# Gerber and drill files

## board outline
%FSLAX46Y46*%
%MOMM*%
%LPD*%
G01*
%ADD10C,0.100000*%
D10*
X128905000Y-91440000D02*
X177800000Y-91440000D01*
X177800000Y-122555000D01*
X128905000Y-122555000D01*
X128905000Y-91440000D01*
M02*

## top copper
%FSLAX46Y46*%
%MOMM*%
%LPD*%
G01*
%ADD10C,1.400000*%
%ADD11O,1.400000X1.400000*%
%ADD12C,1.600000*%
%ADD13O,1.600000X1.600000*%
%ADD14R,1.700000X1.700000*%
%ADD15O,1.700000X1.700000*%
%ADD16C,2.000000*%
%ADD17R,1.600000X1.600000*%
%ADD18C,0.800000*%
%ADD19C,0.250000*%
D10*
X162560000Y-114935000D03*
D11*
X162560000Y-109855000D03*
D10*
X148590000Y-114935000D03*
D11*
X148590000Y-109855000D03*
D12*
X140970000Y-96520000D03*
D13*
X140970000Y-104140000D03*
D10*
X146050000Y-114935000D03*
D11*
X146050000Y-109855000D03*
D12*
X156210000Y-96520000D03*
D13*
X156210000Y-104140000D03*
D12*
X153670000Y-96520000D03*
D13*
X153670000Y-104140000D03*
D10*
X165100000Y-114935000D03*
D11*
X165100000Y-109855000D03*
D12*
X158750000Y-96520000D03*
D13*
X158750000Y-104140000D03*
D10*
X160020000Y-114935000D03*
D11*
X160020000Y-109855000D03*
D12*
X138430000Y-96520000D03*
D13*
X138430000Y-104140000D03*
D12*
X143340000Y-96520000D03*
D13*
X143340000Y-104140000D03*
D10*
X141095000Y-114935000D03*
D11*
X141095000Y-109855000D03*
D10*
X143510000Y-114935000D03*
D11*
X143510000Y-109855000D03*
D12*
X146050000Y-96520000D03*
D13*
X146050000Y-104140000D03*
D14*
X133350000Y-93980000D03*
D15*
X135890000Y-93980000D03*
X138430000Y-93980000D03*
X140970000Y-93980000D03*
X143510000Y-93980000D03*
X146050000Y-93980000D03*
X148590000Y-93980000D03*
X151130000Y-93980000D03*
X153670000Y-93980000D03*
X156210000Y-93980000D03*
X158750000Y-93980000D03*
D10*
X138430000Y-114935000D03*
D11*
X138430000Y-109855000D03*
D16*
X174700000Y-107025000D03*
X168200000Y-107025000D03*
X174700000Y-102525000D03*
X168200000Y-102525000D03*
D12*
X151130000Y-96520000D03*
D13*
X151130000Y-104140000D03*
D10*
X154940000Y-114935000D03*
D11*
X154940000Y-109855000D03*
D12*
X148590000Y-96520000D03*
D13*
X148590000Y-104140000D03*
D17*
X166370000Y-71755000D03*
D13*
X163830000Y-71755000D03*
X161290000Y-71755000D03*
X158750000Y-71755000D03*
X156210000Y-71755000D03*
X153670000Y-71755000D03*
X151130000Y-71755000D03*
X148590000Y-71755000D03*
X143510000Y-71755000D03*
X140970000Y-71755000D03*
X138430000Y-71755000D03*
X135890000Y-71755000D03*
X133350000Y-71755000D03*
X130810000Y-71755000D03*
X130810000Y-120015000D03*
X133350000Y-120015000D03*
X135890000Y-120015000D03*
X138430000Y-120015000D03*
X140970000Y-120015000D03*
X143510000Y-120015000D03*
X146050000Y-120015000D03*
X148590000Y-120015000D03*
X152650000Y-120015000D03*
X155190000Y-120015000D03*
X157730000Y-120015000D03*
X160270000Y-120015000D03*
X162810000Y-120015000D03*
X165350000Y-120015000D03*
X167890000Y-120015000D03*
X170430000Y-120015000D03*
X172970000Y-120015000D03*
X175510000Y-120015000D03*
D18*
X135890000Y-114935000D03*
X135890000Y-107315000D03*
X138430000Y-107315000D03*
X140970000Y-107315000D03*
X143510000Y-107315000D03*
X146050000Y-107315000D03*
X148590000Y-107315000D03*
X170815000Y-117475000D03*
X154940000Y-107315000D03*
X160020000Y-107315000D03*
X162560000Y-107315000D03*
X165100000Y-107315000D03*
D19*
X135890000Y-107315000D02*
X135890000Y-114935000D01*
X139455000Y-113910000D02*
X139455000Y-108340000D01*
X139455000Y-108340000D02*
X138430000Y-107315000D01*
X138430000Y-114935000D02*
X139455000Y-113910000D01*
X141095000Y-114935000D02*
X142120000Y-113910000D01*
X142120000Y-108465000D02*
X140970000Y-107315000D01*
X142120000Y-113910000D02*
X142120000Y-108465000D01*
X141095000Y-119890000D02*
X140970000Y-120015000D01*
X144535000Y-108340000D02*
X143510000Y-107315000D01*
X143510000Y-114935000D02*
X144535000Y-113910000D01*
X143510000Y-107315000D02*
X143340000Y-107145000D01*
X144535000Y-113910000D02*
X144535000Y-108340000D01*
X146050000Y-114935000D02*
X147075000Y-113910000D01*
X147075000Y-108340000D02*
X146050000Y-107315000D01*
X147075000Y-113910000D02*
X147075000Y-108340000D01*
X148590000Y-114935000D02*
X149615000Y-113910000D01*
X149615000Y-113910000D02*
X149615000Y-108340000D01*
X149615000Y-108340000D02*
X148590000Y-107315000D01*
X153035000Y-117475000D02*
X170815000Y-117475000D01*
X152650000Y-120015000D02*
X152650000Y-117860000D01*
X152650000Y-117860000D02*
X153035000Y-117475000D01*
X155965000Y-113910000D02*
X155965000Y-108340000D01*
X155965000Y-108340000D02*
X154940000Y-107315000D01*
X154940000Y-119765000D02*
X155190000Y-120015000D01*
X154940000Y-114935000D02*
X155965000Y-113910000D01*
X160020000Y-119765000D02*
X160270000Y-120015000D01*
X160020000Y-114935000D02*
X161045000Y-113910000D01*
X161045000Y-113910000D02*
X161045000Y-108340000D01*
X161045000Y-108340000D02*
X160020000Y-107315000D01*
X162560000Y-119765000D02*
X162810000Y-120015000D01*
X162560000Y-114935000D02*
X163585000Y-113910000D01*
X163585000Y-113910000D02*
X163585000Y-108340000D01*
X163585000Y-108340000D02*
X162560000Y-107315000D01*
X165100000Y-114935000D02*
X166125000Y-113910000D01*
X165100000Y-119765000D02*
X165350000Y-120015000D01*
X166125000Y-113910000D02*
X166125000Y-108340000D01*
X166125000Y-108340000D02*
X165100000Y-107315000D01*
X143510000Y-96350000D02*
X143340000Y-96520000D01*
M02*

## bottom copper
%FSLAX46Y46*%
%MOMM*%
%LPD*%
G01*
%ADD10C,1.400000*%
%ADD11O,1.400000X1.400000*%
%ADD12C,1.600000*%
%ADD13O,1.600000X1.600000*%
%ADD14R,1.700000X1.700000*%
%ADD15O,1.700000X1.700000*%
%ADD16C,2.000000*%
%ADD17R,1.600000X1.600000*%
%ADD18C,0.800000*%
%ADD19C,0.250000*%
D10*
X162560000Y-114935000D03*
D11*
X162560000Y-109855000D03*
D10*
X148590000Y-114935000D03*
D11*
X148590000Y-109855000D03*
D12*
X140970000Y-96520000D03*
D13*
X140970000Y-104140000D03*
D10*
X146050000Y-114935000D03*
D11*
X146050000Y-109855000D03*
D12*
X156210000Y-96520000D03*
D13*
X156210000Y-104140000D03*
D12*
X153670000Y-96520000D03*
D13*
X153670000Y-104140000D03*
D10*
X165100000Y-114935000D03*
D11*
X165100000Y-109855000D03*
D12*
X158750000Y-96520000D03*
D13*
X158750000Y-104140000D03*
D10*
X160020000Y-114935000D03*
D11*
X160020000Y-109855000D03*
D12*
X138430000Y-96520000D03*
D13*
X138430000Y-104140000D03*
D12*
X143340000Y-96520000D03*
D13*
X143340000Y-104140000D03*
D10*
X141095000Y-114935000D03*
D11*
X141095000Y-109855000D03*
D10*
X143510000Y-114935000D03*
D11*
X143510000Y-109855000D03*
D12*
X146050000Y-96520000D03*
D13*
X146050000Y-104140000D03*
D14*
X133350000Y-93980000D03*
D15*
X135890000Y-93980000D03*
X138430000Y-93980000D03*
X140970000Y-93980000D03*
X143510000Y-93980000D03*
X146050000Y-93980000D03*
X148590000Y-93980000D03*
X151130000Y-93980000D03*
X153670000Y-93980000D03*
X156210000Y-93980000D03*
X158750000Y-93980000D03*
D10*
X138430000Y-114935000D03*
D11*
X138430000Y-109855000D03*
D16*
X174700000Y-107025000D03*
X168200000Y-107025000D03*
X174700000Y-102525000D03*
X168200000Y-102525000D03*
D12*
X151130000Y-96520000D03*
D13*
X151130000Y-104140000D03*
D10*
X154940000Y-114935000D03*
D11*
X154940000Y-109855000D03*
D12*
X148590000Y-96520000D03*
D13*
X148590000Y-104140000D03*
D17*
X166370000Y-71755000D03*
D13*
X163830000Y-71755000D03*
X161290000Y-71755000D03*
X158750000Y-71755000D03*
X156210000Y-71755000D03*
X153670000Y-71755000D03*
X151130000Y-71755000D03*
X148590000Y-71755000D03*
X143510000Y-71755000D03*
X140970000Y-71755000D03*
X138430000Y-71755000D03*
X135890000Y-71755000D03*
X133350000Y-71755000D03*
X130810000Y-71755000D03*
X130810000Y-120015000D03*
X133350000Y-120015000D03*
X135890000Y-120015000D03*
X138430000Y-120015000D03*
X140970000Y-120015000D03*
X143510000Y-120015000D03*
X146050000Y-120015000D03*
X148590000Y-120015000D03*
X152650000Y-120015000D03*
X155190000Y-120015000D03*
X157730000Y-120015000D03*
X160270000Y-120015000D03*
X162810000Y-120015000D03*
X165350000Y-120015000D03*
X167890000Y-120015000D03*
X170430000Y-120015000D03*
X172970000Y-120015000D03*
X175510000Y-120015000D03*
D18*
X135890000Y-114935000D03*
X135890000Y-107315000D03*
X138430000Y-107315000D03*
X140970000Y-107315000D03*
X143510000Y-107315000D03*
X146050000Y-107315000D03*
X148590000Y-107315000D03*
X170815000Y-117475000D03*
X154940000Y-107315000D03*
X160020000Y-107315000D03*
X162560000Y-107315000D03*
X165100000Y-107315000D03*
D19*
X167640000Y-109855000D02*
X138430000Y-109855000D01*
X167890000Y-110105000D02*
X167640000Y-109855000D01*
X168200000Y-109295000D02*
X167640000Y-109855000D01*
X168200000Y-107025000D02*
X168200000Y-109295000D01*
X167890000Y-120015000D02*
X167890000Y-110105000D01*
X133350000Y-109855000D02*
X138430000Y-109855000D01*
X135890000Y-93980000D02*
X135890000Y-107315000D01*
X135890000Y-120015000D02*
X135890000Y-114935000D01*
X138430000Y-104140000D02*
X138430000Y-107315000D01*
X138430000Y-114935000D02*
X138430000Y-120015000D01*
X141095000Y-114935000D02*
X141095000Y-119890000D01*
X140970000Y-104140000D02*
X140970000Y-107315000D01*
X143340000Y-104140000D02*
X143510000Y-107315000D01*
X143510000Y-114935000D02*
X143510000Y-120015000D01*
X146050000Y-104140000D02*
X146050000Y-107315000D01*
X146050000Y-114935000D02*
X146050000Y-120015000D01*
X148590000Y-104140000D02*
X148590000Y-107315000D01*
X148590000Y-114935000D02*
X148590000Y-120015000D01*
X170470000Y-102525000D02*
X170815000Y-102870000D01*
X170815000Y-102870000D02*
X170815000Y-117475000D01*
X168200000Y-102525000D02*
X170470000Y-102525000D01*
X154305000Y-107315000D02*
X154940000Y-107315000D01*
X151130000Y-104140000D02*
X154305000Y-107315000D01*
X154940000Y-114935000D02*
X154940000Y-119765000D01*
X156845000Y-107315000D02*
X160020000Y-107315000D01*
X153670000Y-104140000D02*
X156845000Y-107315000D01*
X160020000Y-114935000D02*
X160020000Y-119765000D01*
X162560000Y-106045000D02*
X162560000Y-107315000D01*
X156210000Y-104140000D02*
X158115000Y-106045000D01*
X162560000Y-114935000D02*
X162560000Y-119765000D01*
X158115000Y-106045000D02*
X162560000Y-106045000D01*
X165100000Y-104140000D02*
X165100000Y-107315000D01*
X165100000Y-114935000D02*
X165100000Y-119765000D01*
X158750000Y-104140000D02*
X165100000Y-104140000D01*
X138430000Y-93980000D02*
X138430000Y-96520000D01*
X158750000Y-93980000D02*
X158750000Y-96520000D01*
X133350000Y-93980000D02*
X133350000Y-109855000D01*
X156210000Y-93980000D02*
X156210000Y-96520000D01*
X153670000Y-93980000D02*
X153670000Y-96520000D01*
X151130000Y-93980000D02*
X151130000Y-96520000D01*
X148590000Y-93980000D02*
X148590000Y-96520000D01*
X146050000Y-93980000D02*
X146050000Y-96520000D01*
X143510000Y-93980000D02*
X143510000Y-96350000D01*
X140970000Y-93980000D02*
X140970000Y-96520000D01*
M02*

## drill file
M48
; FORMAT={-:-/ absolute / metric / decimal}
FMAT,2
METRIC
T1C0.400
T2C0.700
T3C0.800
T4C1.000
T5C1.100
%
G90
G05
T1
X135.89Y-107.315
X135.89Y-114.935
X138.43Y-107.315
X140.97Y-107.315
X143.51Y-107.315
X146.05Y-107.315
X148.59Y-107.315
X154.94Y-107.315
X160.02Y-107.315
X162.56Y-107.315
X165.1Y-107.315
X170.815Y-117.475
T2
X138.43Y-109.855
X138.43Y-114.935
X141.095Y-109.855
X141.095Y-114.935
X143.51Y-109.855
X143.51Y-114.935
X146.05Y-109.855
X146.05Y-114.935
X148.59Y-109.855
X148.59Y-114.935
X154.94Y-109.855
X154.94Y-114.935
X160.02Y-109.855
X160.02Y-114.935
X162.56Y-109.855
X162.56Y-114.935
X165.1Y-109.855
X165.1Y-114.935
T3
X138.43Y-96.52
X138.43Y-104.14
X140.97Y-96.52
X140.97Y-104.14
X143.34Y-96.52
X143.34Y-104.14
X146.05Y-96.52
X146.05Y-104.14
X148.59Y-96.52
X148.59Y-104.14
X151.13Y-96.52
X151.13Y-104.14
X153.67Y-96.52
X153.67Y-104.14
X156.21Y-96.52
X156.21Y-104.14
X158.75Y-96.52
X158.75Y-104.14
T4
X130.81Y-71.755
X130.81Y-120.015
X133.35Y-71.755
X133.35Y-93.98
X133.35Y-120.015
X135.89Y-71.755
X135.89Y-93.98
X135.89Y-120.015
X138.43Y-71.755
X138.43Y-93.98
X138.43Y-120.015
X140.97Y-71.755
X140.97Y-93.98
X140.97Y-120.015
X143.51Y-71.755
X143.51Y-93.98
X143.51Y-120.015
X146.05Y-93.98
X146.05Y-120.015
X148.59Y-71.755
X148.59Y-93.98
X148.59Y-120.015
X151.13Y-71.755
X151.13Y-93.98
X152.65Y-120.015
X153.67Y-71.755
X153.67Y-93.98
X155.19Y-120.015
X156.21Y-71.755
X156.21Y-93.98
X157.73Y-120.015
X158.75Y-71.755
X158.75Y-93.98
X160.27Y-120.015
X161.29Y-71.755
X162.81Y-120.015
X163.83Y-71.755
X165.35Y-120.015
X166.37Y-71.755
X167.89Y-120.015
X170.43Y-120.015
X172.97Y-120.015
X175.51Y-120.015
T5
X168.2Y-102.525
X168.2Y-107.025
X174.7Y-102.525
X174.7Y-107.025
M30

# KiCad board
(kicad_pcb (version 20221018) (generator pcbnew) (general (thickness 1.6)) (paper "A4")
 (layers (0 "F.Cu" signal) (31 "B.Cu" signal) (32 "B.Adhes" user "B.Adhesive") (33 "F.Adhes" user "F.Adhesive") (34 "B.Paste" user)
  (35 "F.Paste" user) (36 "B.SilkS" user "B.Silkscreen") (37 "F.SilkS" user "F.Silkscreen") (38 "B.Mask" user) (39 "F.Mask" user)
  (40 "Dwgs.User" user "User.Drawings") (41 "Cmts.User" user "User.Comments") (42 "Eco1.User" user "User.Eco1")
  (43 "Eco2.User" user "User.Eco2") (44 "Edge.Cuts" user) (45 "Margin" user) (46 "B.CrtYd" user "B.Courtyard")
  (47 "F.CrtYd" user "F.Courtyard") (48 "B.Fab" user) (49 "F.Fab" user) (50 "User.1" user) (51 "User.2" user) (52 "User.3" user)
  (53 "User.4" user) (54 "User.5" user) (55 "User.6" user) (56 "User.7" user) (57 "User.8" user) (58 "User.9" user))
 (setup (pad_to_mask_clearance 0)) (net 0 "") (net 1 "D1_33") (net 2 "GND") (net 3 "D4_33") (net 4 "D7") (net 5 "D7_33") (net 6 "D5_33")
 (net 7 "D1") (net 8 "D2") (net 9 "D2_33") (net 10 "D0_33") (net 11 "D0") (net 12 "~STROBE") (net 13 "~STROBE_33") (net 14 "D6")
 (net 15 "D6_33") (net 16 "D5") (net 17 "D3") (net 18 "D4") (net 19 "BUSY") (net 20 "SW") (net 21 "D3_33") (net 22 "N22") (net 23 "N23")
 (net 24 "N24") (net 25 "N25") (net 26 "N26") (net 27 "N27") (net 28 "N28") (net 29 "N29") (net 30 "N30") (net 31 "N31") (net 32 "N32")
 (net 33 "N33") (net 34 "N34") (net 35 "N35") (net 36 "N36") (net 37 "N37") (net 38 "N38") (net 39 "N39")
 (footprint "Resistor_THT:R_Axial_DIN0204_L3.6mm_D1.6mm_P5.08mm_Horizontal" (layer "F.Cu") (at 162.56 114.935 90)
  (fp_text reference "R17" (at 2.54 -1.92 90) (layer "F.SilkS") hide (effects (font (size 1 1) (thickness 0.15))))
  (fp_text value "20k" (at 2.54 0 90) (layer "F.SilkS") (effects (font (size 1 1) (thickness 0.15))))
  (pad "1" thru_hole circle (at 0 0 90) (size 1.4 1.4) (drill 0.7) (layers "*.Cu" "*.Mask") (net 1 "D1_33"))
  (pad "2" thru_hole oval (at 5.08 0 90) (size 1.4 1.4) (drill 0.7) (layers "*.Cu" "*.Mask") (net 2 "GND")))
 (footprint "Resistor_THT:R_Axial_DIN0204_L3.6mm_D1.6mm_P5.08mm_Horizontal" (layer "F.Cu") (at 148.59 114.935 90)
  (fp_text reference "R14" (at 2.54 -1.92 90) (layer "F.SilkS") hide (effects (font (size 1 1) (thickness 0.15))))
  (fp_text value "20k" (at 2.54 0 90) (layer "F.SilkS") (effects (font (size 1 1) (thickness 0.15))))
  (pad "1" thru_hole circle (at 0 0 90) (size 1.4 1.4) (drill 0.7) (layers "*.Cu" "*.Mask") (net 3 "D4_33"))
  (pad "2" thru_hole oval (at 5.08 0 90) (size 1.4 1.4) (drill 0.7) (layers "*.Cu" "*.Mask") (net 2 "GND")))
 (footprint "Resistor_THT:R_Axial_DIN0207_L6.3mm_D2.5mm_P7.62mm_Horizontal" (layer "F.Cu") (at 140.97 96.52 -90)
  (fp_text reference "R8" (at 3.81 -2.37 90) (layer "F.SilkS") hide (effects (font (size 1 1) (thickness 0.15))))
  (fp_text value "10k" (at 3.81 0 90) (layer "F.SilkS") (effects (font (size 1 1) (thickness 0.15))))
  (pad "1" thru_hole circle (at 0 0 270) (size 1.6 1.6) (drill 0.8) (layers "*.Cu" "*.Mask") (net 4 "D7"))
  (pad "2" thru_hole oval (at 7.62 0 270) (size 1.6 1.6) (drill 0.8) (layers "*.Cu" "*.Mask") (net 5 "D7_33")))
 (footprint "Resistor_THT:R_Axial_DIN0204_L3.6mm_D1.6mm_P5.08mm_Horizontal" (layer "F.Cu") (at 146.05 114.935 90)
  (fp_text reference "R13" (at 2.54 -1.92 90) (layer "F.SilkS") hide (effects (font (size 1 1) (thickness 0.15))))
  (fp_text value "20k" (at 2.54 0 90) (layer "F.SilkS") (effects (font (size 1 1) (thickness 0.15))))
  (pad "1" thru_hole circle (at 0 0 90) (size 1.4 1.4) (drill 0.7) (layers "*.Cu" "*.Mask") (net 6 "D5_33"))
  (pad "2" thru_hole oval (at 5.08 0 90) (size 1.4 1.4) (drill 0.7) (layers "*.Cu" "*.Mask") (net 2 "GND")))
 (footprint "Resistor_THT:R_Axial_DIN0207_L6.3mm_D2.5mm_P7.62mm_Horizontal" (layer "F.Cu") (at 156.21 96.52 -90)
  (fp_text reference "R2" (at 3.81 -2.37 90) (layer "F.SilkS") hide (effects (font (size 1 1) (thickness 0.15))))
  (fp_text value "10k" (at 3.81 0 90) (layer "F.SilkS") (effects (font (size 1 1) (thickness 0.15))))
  (pad "1" thru_hole circle (at 0 0 270) (size 1.6 1.6) (drill 0.8) (layers "*.Cu" "*.Mask") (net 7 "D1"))
  (pad "2" thru_hole oval (at 7.62 0 270) (size 1.6 1.6) (drill 0.8) (layers "*.Cu" "*.Mask") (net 1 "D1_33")))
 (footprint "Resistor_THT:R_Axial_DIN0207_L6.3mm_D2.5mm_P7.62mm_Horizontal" (layer "F.Cu") (at 153.67 96.52 -90)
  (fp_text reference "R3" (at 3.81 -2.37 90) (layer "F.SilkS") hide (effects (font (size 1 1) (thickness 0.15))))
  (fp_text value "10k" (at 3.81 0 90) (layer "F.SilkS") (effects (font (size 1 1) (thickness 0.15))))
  (pad "1" thru_hole circle (at 0 0 270) (size 1.6 1.6) (drill 0.8) (layers "*.Cu" "*.Mask") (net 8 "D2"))
  (pad "2" thru_hole oval (at 7.62 0 270) (size 1.6 1.6) (drill 0.8) (layers "*.Cu" "*.Mask") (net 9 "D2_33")))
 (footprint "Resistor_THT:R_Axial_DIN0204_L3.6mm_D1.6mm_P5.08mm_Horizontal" (layer "F.Cu") (at 165.1 114.935 90)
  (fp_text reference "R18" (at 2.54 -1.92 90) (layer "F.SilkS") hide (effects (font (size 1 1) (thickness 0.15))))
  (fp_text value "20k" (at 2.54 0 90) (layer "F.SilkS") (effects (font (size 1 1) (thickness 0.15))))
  (pad "1" thru_hole circle (at 0 0 90) (size 1.4 1.4) (drill 0.7) (layers "*.Cu" "*.Mask") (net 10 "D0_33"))
  (pad "2" thru_hole oval (at 5.08 0 90) (size 1.4 1.4) (drill 0.7) (layers "*.Cu" "*.Mask") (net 2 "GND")))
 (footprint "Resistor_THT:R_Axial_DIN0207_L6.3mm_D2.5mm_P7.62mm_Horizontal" (layer "F.Cu") (at 158.75 96.52 -90)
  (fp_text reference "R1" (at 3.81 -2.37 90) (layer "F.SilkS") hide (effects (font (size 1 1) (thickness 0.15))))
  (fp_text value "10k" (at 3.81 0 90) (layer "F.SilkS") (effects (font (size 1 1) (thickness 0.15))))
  (pad "1" thru_hole circle (at 0 0 270) (size 1.6 1.6) (drill 0.8) (layers "*.Cu" "*.Mask") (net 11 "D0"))
  (pad "2" thru_hole oval (at 7.62 0 270) (size 1.6 1.6) (drill 0.8) (layers "*.Cu" "*.Mask") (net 10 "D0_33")))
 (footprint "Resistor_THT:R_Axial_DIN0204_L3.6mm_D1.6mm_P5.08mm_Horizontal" (layer "F.Cu") (at 160.02 114.935 90)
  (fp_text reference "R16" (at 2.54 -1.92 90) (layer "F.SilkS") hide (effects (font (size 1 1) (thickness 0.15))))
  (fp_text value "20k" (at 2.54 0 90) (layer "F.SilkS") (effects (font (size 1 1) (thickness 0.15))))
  (pad "1" thru_hole circle (at 0 0 90) (size 1.4 1.4) (drill 0.7) (layers "*.Cu" "*.Mask") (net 9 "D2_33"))
  (pad "2" thru_hole oval (at 5.08 0 90) (size 1.4 1.4) (drill 0.7) (layers "*.Cu" "*.Mask") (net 2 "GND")))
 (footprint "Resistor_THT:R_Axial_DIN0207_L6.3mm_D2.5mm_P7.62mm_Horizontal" (layer "F.Cu") (at 138.43 96.52 -90)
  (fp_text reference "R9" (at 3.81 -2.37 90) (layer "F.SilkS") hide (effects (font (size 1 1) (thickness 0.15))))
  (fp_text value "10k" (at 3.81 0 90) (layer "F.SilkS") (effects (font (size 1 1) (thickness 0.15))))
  (pad "1" thru_hole circle (at 0 0 270) (size 1.6 1.6) (drill 0.8) (layers "*.Cu" "*.Mask") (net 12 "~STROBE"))
  (pad "2" thru_hole oval (at 7.62 0 270) (size 1.6 1.6) (drill 0.8) (layers "*.Cu" "*.Mask") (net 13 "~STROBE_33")))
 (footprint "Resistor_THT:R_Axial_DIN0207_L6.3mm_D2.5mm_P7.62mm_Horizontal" (layer "F.Cu") (at 143.34 96.52 -90)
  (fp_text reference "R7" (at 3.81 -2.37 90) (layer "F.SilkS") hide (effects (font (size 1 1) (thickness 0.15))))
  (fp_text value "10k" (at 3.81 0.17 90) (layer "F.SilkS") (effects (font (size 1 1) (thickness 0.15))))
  (pad "1" thru_hole circle (at 0 0 270) (size 1.6 1.6) (drill 0.8) (layers "*.Cu" "*.Mask") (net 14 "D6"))
  (pad "2" thru_hole oval (at 7.62 0 270) (size 1.6 1.6) (drill 0.8) (layers "*.Cu" "*.Mask") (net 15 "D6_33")))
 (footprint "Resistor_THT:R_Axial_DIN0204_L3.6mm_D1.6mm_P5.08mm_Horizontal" (layer "F.Cu") (at 141.095 114.935 90)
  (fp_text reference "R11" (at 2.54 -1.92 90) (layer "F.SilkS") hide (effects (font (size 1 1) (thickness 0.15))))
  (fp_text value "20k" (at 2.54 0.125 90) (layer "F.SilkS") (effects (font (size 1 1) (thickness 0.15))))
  (pad "1" thru_hole circle (at 0 0 90) (size 1.4 1.4) (drill 0.7) (layers "*.Cu" "*.Mask") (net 5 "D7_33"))
  (pad "2" thru_hole oval (at 5.08 0 90) (size 1.4 1.4) (drill 0.7) (layers "*.Cu" "*.Mask") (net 2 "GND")))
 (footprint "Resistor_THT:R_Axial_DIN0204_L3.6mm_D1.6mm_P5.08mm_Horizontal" (layer "F.Cu") (at 143.51 114.935 90)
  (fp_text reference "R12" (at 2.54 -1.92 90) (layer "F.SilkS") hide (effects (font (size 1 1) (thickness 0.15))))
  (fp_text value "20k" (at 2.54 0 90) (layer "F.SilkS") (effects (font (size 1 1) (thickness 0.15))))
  (pad "1" thru_hole circle (at 0 0 90) (size 1.4 1.4) (drill 0.7) (layers "*.Cu" "*.Mask") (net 15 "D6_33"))
  (pad "2" thru_hole oval (at 5.08 0 90) (size 1.4 1.4) (drill 0.7) (layers "*.Cu" "*.Mask") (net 2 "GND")))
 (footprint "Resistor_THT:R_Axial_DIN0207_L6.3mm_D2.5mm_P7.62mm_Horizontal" (layer "F.Cu") (at 146.05 96.52 -90)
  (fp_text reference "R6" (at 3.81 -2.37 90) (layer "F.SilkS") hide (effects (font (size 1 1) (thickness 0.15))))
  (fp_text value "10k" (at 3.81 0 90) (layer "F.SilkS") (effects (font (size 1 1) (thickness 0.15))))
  (pad "1" thru_hole circle (at 0 0 270) (size 1.6 1.6) (drill 0.8) (layers "*.Cu" "*.Mask") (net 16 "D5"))
  (pad "2" thru_hole oval (at 7.62 0 270) (size 1.6 1.6) (drill 0.8) (layers "*.Cu" "*.Mask") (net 6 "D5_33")))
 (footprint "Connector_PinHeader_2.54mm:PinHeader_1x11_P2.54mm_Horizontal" (layer "F.Cu") (at 133.35 93.98 90)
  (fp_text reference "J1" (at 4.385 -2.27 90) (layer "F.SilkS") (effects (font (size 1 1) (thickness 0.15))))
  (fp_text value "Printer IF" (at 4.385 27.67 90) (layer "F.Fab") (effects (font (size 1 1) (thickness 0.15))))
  (pad "1" thru_hole rect (at 0 0 90) (size 1.7 1.7) (drill 1) (layers "*.Cu" "*.Mask") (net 11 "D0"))
  (pad "2" thru_hole oval (at 0 2.54 90) (size 1.7 1.7) (drill 1) (layers "*.Cu" "*.Mask") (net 7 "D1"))
  (pad "3" thru_hole oval (at 0 5.08 90) (size 1.7 1.7) (drill 1) (layers "*.Cu" "*.Mask") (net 8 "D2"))
  (pad "4" thru_hole oval (at 0 7.62 90) (size 1.7 1.7) (drill 1) (layers "*.Cu" "*.Mask") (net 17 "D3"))
  (pad "5" thru_hole oval (at 0 10.16 90) (size 1.7 1.7) (drill 1) (layers "*.Cu" "*.Mask") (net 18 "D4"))
  (pad "6" thru_hole oval (at 0 12.7 90) (size 1.7 1.7) (drill 1) (layers "*.Cu" "*.Mask") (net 16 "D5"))
  (pad "7" thru_hole oval (at 0 15.24 90) (size 1.7 1.7) (drill 1) (layers "*.Cu" "*.Mask") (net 14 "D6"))
  (pad "8" thru_hole oval (at 0 17.78 90) (size 1.7 1.7) (drill 1) (layers "*.Cu" "*.Mask") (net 4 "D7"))
  (pad "9" thru_hole oval (at 0 20.32 90) (size 1.7 1.7) (drill 1) (layers "*.Cu" "*.Mask") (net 12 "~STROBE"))
  (pad "10" thru_hole oval (at 0 22.86 90) (size 1.7 1.7) (drill 1) (layers "*.Cu" "*.Mask") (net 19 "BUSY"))
  (pad "11" thru_hole oval (at 0 25.4 90) (size 1.7 1.7) (drill 1) (layers "*.Cu" "*.Mask") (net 2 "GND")))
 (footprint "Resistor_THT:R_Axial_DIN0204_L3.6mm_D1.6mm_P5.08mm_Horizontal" (layer "F.Cu") (at 138.43 114.935 90)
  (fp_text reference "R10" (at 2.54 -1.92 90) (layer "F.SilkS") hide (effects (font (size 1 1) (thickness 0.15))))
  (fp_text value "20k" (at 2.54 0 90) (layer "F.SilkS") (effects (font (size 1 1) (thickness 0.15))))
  (pad "1" thru_hole circle (at 0 0 90) (size 1.4 1.4) (drill 0.7) (layers "*.Cu" "*.Mask") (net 13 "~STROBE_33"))
  (pad "2" thru_hole oval (at 5.08 0 90) (size 1.4 1.4) (drill 0.7) (layers "*.Cu" "*.Mask") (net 2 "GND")))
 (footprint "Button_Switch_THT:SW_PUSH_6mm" (layer "F.Cu") (at 174.7 107.025 180)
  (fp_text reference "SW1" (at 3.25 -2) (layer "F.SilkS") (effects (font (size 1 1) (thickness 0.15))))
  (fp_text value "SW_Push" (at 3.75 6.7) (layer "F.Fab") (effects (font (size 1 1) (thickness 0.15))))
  (pad "1" thru_hole circle (at 0 0 270) (size 2 2) (drill 1.1) (layers "*.Cu" "*.Mask") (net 2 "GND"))
  (pad "1" thru_hole circle (at 6.5 0 270) (size 2 2) (drill 1.1) (layers "*.Cu" "*.Mask") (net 2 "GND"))
  (pad "2" thru_hole circle (at 0 4.5 270) (size 2 2) (drill 1.1) (layers "*.Cu" "*.Mask") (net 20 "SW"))
  (pad "2" thru_hole circle (at 6.5 4.5 270) (size 2 2) (drill 1.1) (layers "*.Cu" "*.Mask") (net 20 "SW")))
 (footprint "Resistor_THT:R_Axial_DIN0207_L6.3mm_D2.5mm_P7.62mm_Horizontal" (layer "F.Cu") (at 151.13 96.52 -90)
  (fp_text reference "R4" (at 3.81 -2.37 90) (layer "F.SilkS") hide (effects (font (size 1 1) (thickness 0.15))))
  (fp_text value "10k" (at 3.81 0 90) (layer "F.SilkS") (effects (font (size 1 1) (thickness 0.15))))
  (pad "1" thru_hole circle (at 0 0 270) (size 1.6 1.6) (drill 0.8) (layers "*.Cu" "*.Mask") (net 17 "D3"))
  (pad "2" thru_hole oval (at 7.62 0 270) (size 1.6 1.6) (drill 0.8) (layers "*.Cu" "*.Mask") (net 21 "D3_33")))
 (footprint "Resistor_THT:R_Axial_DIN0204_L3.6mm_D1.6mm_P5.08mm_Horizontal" (layer "F.Cu") (at 154.94 114.935 90)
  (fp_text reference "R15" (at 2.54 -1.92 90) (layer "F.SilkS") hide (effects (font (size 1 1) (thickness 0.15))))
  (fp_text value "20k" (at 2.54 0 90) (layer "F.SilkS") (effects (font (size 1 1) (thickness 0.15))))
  (pad "1" thru_hole circle (at 0 0 90) (size 1.4 1.4) (drill 0.7) (layers "*.Cu" "*.Mask") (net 21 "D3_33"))
  (pad "2" thru_hole oval (at 5.08 0 90) (size 1.4 1.4) (drill 0.7) (layers "*.Cu" "*.Mask") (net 2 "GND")))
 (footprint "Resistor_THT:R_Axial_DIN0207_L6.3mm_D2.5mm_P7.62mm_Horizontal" (layer "F.Cu") (at 148.59 96.52 -90)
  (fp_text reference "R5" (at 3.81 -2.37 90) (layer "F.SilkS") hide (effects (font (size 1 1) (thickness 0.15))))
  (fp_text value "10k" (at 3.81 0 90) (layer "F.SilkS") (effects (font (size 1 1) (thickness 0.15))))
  (pad "1" thru_hole circle (at 0 0 270) (size 1.6 1.6) (drill 0.8) (layers "*.Cu" "*.Mask") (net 18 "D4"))
  (pad "2" thru_hole oval (at 7.62 0 270) (size 1.6 1.6) (drill 0.8) (layers "*.Cu" "*.Mask") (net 3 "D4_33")))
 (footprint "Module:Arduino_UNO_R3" (layer "B.Cu") (at 166.37 71.755 180)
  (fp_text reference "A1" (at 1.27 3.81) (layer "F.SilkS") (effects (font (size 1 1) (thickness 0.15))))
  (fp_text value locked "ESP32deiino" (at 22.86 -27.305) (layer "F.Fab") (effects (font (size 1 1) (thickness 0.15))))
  (pad "1" thru_hole rect (at 0 0 90) (size 1.6 1.6) (drill 1) (layers "*.Cu" "*.Mask") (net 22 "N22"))
  (pad "2" thru_hole oval (at 2.54 0 90) (size 1.6 1.6) (drill 1) (layers "*.Cu" "*.Mask") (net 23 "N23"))
  (pad "3" thru_hole oval (at 5.08 0 90) (size 1.6 1.6) (drill 1) (layers "*.Cu" "*.Mask") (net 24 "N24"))
  (pad "4" thru_hole oval (at 7.62 0 90) (size 1.6 1.6) (drill 1) (layers "*.Cu" "*.Mask") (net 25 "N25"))
  (pad "5" thru_hole oval (at 10.16 0 90) (size 1.6 1.6) (drill 1) (layers "*.Cu" "*.Mask") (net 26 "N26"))
  (pad "6" thru_hole oval (at 12.7 0 90) (size 1.6 1.6) (drill 1) (layers "*.Cu" "*.Mask") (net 2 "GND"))
  (pad "7" thru_hole oval (at 15.24 0 90) (size 1.6 1.6) (drill 1) (layers "*.Cu" "*.Mask") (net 2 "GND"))
  (pad "8" thru_hole oval (at 17.78 0 90) (size 1.6 1.6) (drill 1) (layers "*.Cu" "*.Mask") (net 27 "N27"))
  (pad "9" thru_hole oval (at 22.86 0 90) (size 1.6 1.6) (drill 1) (layers "*.Cu" "*.Mask") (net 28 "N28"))
  (pad "10" thru_hole oval (at 25.4 0 90) (size 1.6 1.6) (drill 1) (layers "*.Cu" "*.Mask") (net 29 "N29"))
  (pad "11" thru_hole oval (at 27.94 0 90) (size 1.6 1.6) (drill 1) (layers "*.Cu" "*.Mask") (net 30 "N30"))
  (pad "12" thru_hole oval (at 30.48 0 90) (size 1.6 1.6) (drill 1) (layers "*.Cu" "*.Mask") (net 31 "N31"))
  (pad "13" thru_hole oval (at 33.02 0 90) (size 1.6 1.6) (drill 1) (layers "*.Cu" "*.Mask") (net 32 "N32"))
  (pad "14" thru_hole oval (at 35.56 0 90) (size 1.6 1.6) (drill 1) (layers "*.Cu" "*.Mask") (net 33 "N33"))
  (pad "15" thru_hole oval (at 35.56 -48.26 90) (size 1.6 1.6) (drill 1) (layers "*.Cu" "*.Mask") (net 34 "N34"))
  (pad "16" thru_hole oval (at 33.02 -48.26 90) (size 1.6 1.6) (drill 1) (layers "*.Cu" "*.Mask") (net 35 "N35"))
  (pad "17" thru_hole oval (at 30.48 -48.26 90) (size 1.6 1.6) (drill 1) (layers "*.Cu" "*.Mask") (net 19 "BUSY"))
  (pad "18" thru_hole oval (at 27.94 -48.26 90) (size 1.6 1.6) (drill 1) (layers "*.Cu" "*.Mask") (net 13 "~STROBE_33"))
  (pad "19" thru_hole oval (at 25.4 -48.26 90) (size 1.6 1.6) (drill 1) (layers "*.Cu" "*.Mask") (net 5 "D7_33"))
  (pad "20" thru_hole oval (at 22.86 -48.26 90) (size 1.6 1.6) (drill 1) (layers "*.Cu" "*.Mask") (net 15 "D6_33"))
  (pad "21" thru_hole oval (at 20.32 -48.26 90) (size 1.6 1.6) (drill 1) (layers "*.Cu" "*.Mask") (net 6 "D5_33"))
  (pad "22" thru_hole oval (at 17.78 -48.26 90) (size 1.6 1.6) (drill 1) (layers "*.Cu" "*.Mask") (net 3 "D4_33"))
  (pad "23" thru_hole oval (at 13.72 -48.26 90) (size 1.6 1.6) (drill 1) (layers "*.Cu" "*.Mask") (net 20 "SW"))
  (pad "24" thru_hole oval (at 11.18 -48.26 90) (size 1.6 1.6) (drill 1) (layers "*.Cu" "*.Mask") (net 21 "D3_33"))
  (pad "25" thru_hole oval (at 8.64 -48.26 90) (size 1.6 1.6) (drill 1) (layers "*.Cu" "*.Mask") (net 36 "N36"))
  (pad "26" thru_hole oval (at 6.1 -48.26 90) (size 1.6 1.6) (drill 1) (layers "*.Cu" "*.Mask") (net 9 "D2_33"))
  (pad "27" thru_hole oval (at 3.56 -48.26 90) (size 1.6 1.6) (drill 1) (layers "*.Cu" "*.Mask") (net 1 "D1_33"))
  (pad "28" thru_hole oval (at 1.02 -48.26 90) (size 1.6 1.6) (drill 1) (layers "*.Cu" "*.Mask") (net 10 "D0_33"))
  (pad "29" thru_hole oval (at -1.52 -48.26 90) (size 1.6 1.6) (drill 1) (layers "*.Cu" "*.Mask") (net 2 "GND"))
  (pad "30" thru_hole oval (at -4.06 -48.26 90) (size 1.6 1.6) (drill 1) (layers "*.Cu" "*.Mask") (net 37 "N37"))
  (pad "31" thru_hole oval (at -6.6 -48.26 90) (size 1.6 1.6) (drill 1) (layers "*.Cu" "*.Mask") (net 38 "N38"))
  (pad "32" thru_hole oval (at -9.14 -48.26 90) (size 1.6 1.6) (drill 1) (layers "*.Cu" "*.Mask") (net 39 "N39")))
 (gr_rect (start 128.905 91.44) (end 177.8 122.555) (stroke (width 0.1) (type default)) (fill none) (layer "Edge.Cuts"))
 (segment (start 167.64 109.855) (end 138.43 109.855) (width 0.25) (layer "B.Cu") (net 2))
 (segment (start 167.89 110.105) (end 167.64 109.855) (width 0.25) (layer "B.Cu") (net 2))
 (segment (start 168.2 109.295) (end 167.64 109.855) (width 0.25) (layer "B.Cu") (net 2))
 (segment (start 168.2 107.025) (end 168.2 109.295) (width 0.25) (layer "B.Cu") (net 2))
 (segment (start 167.89 120.015) (end 167.89 110.105) (width 0.25) (layer "B.Cu") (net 2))
 (segment (start 133.35 109.855) (end 138.43 109.855) (width 0.25) (layer "B.Cu") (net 2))
 (segment (start 135.89 107.315) (end 135.89 114.935) (width 0.25) (layer "F.Cu") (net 19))
 (via (at 135.89 114.935) (size 0.8) (drill 0.4) (layers "F.Cu" "B.Cu") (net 19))
 (via (at 135.89 107.315) (size 0.8) (drill 0.4) (layers "F.Cu" "B.Cu") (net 19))
 (segment (start 135.89 93.98) (end 135.89 107.315) (width 0.25) (layer "B.Cu") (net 19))
 (segment (start 135.89 120.015) (end 135.89 114.935) (width 0.25) (layer "B.Cu") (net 19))
 (segment (start 139.455 113.91) (end 139.455 108.34) (width 0.25) (layer "F.Cu") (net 13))
 (segment (start 139.455 108.34) (end 138.43 107.315) (width 0.25) (layer "F.Cu") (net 13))
 (segment (start 138.43 114.935) (end 139.455 113.91) (width 0.25) (layer "F.Cu") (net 13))
 (via (at 138.43 107.315) (size 0.8) (drill 0.4) (layers "F.Cu" "B.Cu") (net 13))
 (segment (start 138.43 104.14) (end 138.43 107.315) (width 0.25) (layer "B.Cu") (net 13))
 (segment (start 138.43 114.935) (end 138.43 120.015) (width 0.25) (layer "B.Cu") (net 13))
 (segment (start 141.095 114.935) (end 142.12 113.91) (width 0.25) (layer "F.Cu") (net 5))
 (segment (start 142.12 108.465) (end 140.97 107.315) (width 0.25) (layer "F.Cu") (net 5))
 (segment (start 142.12 113.91) (end 142.12 108.465) (width 0.25) (layer "F.Cu") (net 5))
 (segment (start 141.095 119.89) (end 140.97 120.015) (width 0.25) (layer "F.Cu") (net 5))
 (via (at 140.97 107.315) (size 0.8) (drill 0.4) (layers "F.Cu" "B.Cu") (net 5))
 (segment (start 141.095 114.935) (end 141.095 119.89) (width 0.25) (layer "B.Cu") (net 5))
 (segment (start 140.97 104.14) (end 140.97 107.315) (width 0.25) (layer "B.Cu") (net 5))
 (segment (start 144.535 108.34) (end 143.51 107.315) (width 0.25) (layer "F.Cu") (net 15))
 (segment (start 143.51 114.935) (end 144.535 113.91) (width 0.25) (layer "F.Cu") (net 15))
 (segment (start 143.51 107.315) (end 143.34 107.145) (width 0.25) (layer "F.Cu") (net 15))
 (segment (start 144.535 113.91) (end 144.535 108.34) (width 0.25) (layer "F.Cu") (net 15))
 (via (at 143.51 107.315) (size 0.8) (drill 0.4) (layers "F.Cu" "B.Cu") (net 15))
 (segment (start 143.34 104.14) (end 143.51 107.315) (width 0.25) (layer "B.Cu") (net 15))
 (segment (start 143.51 114.935) (end 143.51 120.015) (width 0.25) (layer "B.Cu") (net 15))
 (segment (start 146.05 114.935) (end 147.075 113.91) (width 0.25) (layer "F.Cu") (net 6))
 (segment (start 147.075 108.34) (end 146.05 107.315) (width 0.25) (layer "F.Cu") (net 6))
 (segment (start 147.075 113.91) (end 147.075 108.34) (width 0.25) (layer "F.Cu") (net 6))
 (via (at 146.05 107.315) (size 0.8) (drill 0.4) (layers "F.Cu" "B.Cu") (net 6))
 (segment (start 146.05 104.14) (end 146.05 107.315) (width 0.25) (layer "B.Cu") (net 6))
 (segment (start 146.05 114.935) (end 146.05 120.015) (width 0.25) (layer "B.Cu") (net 6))
 (segment (start 148.59 114.935) (end 149.615 113.91) (width 0.25) (layer "F.Cu") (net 3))
 (segment (start 149.615 113.91) (end 149.615 108.34) (width 0.25) (layer "F.Cu") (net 3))
 (segment (start 149.615 108.34) (end 148.59 107.315) (width 0.25) (layer "F.Cu") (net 3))
 (via (at 148.59 107.315) (size 0.8) (drill 0.4) (layers "F.Cu" "B.Cu") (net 3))
 (segment (start 148.59 104.14) (end 148.59 107.315) (width 0.25) (layer "B.Cu") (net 3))
 (segment (start 148.59 114.935) (end 148.59 120.015) (width 0.25) (layer "B.Cu") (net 3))
 (segment (start 153.035 117.475) (end 170.815 117.475) (width 0.25) (layer "F.Cu") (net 20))
 (segment (start 152.65 120.015) (end 152.65 117.86) (width 0.25) (layer "F.Cu") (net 20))
 (segment (start 152.65 117.86) (end 153.035 117.475) (width 0.25) (layer "F.Cu") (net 20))
 (via (at 170.815 117.475) (size 0.8) (drill 0.4) (layers "F.Cu" "B.Cu") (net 20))
 (segment (start 170.47 102.525) (end 170.815 102.87) (width 0.25) (layer "B.Cu") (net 20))
 (segment (start 170.815 102.87) (end 170.815 117.475) (width 0.25) (layer "B.Cu") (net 20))
 (segment (start 168.2 102.525) (end 170.47 102.525) (width 0.25) (layer "B.Cu") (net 20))
 (segment (start 155.965 113.91) (end 155.965 108.34) (width 0.25) (layer "F.Cu") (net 21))
 (segment (start 155.965 108.34) (end 154.94 107.315) (width 0.25) (layer "F.Cu") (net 21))
 (segment (start 154.94 119.765) (end 155.19 120.015) (width 0.25) (layer "F.Cu") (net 21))
 (segment (start 154.94 114.935) (end 155.965 113.91) (width 0.25) (layer "F.Cu") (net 21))
 (via (at 154.94 107.315) (size 0.8) (drill 0.4) (layers "F.Cu" "B.Cu") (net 21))
 (segment (start 154.305 107.315) (end 154.94 107.315) (width 0.25) (layer "B.Cu") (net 21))
 (segment (start 151.13 104.14) (end 154.305 107.315) (width 0.25) (layer "B.Cu") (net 21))
 (segment (start 154.94 114.935) (end 154.94 119.765) (width 0.25) (layer "B.Cu") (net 21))
 (segment (start 160.02 119.765) (end 160.27 120.015) (width 0.25) (layer "F.Cu") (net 9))
 (segment (start 160.02 114.935) (end 161.045 113.91) (width 0.25) (layer "F.Cu") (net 9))
 (segment (start 161.045 113.91) (end 161.045 108.34) (width 0.25) (layer "F.Cu") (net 9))
 (segment (start 161.045 108.34) (end 160.02 107.315) (width 0.25) (layer "F.Cu") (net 9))
 (via (at 160.02 107.315) (size 0.8) (drill 0.4) (layers "F.Cu" "B.Cu") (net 9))
 (segment (start 156.845 107.315) (end 160.02 107.315) (width 0.25) (layer "B.Cu") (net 9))
 (segment (start 153.67 104.14) (end 156.845 107.315) (width 0.25) (layer "B.Cu") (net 9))
 (segment (start 160.02 114.935) (end 160.02 119.765) (width 0.25) (layer "B.Cu") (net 9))
 (segment (start 162.56 119.765) (end 162.81 120.015) (width 0.25) (layer "F.Cu") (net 1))
 (segment (start 162.56 114.935) (end 163.585 113.91) (width 0.25) (layer "F.Cu") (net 1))
 (segment (start 163.585 113.91) (end 163.585 108.34) (width 0.25) (layer "F.Cu") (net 1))
 (segment (start 163.585 108.34) (end 162.56 107.315) (width 0.25) (layer "F.Cu") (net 1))
 (via (at 162.56 107.315) (size 0.8) (drill 0.4) (layers "F.Cu" "B.Cu") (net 1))
 (segment (start 162.56 106.045) (end 162.56 107.315) (width 0.25) (layer "B.Cu") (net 1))
 (segment (start 156.21 104.14) (end 158.115 106.045) (width 0.25) (layer "B.Cu") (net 1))
 (segment (start 162.56 114.935) (end 162.56 119.765) (width 0.25) (layer "B.Cu") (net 1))
 (segment (start 158.115 106.045) (end 162.56 106.045) (width 0.25) (layer "B.Cu") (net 1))
 (segment (start 165.1 114.935) (end 166.125 113.91) (width 0.25) (layer "F.Cu") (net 10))
 (segment (start 165.1 119.765) (end 165.35 120.015) (width 0.25) (layer "F.Cu") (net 10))
 (segment (start 166.125 113.91) (end 166.125 108.34) (width 0.25) (layer "F.Cu") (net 10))
 (segment (start 166.125 108.34) (end 165.1 107.315) (width 0.25) (layer "F.Cu") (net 10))
 (via (at 165.1 107.315) (size 0.8) (drill 0.4) (layers "F.Cu" "B.Cu") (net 10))
 (segment (start 165.1 104.14) (end 165.1 107.315) (width 0.25) (layer "B.Cu") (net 10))
 (segment (start 165.1 114.935) (end 165.1 119.765) (width 0.25) (layer "B.Cu") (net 10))
 (segment (start 158.75 104.14) (end 165.1 104.14) (width 0.25) (layer "B.Cu") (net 10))
 (segment (start 138.43 93.98) (end 138.43 96.52) (width 0.25) (layer "B.Cu") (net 12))
 (segment (start 158.75 93.98) (end 158.75 96.52) (width 0.25) (layer "B.Cu") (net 11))
 (segment (start 133.35 93.98) (end 133.35 109.855) (width 0.25) (layer "B.Cu") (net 11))
 (segment (start 156.21 93.98) (end 156.21 96.52) (width 0.25) (layer "B.Cu") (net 7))
 (segment (start 153.67 93.98) (end 153.67 96.52) (width 0.25) (layer "B.Cu") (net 8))
 (segment (start 151.13 93.98) (end 151.13 96.52) (width 0.25) (layer "B.Cu") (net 17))
 (segment (start 148.59 93.98) (end 148.59 96.52) (width 0.25) (layer "B.Cu") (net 18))
 (segment (start 146.05 93.98) (end 146.05 96.52) (width 0.25) (layer "B.Cu") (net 16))
 (segment (start 143.51 96.35) (end 143.34 96.52) (width 0.25) (layer "F.Cu") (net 14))
 (segment (start 143.51 93.98) (end 143.51 96.35) (width 0.25) (layer "B.Cu") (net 14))
 (segment (start 140.97 93.98) (end 140.97 96.52) (width 0.25) (layer "B.Cu") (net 4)))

